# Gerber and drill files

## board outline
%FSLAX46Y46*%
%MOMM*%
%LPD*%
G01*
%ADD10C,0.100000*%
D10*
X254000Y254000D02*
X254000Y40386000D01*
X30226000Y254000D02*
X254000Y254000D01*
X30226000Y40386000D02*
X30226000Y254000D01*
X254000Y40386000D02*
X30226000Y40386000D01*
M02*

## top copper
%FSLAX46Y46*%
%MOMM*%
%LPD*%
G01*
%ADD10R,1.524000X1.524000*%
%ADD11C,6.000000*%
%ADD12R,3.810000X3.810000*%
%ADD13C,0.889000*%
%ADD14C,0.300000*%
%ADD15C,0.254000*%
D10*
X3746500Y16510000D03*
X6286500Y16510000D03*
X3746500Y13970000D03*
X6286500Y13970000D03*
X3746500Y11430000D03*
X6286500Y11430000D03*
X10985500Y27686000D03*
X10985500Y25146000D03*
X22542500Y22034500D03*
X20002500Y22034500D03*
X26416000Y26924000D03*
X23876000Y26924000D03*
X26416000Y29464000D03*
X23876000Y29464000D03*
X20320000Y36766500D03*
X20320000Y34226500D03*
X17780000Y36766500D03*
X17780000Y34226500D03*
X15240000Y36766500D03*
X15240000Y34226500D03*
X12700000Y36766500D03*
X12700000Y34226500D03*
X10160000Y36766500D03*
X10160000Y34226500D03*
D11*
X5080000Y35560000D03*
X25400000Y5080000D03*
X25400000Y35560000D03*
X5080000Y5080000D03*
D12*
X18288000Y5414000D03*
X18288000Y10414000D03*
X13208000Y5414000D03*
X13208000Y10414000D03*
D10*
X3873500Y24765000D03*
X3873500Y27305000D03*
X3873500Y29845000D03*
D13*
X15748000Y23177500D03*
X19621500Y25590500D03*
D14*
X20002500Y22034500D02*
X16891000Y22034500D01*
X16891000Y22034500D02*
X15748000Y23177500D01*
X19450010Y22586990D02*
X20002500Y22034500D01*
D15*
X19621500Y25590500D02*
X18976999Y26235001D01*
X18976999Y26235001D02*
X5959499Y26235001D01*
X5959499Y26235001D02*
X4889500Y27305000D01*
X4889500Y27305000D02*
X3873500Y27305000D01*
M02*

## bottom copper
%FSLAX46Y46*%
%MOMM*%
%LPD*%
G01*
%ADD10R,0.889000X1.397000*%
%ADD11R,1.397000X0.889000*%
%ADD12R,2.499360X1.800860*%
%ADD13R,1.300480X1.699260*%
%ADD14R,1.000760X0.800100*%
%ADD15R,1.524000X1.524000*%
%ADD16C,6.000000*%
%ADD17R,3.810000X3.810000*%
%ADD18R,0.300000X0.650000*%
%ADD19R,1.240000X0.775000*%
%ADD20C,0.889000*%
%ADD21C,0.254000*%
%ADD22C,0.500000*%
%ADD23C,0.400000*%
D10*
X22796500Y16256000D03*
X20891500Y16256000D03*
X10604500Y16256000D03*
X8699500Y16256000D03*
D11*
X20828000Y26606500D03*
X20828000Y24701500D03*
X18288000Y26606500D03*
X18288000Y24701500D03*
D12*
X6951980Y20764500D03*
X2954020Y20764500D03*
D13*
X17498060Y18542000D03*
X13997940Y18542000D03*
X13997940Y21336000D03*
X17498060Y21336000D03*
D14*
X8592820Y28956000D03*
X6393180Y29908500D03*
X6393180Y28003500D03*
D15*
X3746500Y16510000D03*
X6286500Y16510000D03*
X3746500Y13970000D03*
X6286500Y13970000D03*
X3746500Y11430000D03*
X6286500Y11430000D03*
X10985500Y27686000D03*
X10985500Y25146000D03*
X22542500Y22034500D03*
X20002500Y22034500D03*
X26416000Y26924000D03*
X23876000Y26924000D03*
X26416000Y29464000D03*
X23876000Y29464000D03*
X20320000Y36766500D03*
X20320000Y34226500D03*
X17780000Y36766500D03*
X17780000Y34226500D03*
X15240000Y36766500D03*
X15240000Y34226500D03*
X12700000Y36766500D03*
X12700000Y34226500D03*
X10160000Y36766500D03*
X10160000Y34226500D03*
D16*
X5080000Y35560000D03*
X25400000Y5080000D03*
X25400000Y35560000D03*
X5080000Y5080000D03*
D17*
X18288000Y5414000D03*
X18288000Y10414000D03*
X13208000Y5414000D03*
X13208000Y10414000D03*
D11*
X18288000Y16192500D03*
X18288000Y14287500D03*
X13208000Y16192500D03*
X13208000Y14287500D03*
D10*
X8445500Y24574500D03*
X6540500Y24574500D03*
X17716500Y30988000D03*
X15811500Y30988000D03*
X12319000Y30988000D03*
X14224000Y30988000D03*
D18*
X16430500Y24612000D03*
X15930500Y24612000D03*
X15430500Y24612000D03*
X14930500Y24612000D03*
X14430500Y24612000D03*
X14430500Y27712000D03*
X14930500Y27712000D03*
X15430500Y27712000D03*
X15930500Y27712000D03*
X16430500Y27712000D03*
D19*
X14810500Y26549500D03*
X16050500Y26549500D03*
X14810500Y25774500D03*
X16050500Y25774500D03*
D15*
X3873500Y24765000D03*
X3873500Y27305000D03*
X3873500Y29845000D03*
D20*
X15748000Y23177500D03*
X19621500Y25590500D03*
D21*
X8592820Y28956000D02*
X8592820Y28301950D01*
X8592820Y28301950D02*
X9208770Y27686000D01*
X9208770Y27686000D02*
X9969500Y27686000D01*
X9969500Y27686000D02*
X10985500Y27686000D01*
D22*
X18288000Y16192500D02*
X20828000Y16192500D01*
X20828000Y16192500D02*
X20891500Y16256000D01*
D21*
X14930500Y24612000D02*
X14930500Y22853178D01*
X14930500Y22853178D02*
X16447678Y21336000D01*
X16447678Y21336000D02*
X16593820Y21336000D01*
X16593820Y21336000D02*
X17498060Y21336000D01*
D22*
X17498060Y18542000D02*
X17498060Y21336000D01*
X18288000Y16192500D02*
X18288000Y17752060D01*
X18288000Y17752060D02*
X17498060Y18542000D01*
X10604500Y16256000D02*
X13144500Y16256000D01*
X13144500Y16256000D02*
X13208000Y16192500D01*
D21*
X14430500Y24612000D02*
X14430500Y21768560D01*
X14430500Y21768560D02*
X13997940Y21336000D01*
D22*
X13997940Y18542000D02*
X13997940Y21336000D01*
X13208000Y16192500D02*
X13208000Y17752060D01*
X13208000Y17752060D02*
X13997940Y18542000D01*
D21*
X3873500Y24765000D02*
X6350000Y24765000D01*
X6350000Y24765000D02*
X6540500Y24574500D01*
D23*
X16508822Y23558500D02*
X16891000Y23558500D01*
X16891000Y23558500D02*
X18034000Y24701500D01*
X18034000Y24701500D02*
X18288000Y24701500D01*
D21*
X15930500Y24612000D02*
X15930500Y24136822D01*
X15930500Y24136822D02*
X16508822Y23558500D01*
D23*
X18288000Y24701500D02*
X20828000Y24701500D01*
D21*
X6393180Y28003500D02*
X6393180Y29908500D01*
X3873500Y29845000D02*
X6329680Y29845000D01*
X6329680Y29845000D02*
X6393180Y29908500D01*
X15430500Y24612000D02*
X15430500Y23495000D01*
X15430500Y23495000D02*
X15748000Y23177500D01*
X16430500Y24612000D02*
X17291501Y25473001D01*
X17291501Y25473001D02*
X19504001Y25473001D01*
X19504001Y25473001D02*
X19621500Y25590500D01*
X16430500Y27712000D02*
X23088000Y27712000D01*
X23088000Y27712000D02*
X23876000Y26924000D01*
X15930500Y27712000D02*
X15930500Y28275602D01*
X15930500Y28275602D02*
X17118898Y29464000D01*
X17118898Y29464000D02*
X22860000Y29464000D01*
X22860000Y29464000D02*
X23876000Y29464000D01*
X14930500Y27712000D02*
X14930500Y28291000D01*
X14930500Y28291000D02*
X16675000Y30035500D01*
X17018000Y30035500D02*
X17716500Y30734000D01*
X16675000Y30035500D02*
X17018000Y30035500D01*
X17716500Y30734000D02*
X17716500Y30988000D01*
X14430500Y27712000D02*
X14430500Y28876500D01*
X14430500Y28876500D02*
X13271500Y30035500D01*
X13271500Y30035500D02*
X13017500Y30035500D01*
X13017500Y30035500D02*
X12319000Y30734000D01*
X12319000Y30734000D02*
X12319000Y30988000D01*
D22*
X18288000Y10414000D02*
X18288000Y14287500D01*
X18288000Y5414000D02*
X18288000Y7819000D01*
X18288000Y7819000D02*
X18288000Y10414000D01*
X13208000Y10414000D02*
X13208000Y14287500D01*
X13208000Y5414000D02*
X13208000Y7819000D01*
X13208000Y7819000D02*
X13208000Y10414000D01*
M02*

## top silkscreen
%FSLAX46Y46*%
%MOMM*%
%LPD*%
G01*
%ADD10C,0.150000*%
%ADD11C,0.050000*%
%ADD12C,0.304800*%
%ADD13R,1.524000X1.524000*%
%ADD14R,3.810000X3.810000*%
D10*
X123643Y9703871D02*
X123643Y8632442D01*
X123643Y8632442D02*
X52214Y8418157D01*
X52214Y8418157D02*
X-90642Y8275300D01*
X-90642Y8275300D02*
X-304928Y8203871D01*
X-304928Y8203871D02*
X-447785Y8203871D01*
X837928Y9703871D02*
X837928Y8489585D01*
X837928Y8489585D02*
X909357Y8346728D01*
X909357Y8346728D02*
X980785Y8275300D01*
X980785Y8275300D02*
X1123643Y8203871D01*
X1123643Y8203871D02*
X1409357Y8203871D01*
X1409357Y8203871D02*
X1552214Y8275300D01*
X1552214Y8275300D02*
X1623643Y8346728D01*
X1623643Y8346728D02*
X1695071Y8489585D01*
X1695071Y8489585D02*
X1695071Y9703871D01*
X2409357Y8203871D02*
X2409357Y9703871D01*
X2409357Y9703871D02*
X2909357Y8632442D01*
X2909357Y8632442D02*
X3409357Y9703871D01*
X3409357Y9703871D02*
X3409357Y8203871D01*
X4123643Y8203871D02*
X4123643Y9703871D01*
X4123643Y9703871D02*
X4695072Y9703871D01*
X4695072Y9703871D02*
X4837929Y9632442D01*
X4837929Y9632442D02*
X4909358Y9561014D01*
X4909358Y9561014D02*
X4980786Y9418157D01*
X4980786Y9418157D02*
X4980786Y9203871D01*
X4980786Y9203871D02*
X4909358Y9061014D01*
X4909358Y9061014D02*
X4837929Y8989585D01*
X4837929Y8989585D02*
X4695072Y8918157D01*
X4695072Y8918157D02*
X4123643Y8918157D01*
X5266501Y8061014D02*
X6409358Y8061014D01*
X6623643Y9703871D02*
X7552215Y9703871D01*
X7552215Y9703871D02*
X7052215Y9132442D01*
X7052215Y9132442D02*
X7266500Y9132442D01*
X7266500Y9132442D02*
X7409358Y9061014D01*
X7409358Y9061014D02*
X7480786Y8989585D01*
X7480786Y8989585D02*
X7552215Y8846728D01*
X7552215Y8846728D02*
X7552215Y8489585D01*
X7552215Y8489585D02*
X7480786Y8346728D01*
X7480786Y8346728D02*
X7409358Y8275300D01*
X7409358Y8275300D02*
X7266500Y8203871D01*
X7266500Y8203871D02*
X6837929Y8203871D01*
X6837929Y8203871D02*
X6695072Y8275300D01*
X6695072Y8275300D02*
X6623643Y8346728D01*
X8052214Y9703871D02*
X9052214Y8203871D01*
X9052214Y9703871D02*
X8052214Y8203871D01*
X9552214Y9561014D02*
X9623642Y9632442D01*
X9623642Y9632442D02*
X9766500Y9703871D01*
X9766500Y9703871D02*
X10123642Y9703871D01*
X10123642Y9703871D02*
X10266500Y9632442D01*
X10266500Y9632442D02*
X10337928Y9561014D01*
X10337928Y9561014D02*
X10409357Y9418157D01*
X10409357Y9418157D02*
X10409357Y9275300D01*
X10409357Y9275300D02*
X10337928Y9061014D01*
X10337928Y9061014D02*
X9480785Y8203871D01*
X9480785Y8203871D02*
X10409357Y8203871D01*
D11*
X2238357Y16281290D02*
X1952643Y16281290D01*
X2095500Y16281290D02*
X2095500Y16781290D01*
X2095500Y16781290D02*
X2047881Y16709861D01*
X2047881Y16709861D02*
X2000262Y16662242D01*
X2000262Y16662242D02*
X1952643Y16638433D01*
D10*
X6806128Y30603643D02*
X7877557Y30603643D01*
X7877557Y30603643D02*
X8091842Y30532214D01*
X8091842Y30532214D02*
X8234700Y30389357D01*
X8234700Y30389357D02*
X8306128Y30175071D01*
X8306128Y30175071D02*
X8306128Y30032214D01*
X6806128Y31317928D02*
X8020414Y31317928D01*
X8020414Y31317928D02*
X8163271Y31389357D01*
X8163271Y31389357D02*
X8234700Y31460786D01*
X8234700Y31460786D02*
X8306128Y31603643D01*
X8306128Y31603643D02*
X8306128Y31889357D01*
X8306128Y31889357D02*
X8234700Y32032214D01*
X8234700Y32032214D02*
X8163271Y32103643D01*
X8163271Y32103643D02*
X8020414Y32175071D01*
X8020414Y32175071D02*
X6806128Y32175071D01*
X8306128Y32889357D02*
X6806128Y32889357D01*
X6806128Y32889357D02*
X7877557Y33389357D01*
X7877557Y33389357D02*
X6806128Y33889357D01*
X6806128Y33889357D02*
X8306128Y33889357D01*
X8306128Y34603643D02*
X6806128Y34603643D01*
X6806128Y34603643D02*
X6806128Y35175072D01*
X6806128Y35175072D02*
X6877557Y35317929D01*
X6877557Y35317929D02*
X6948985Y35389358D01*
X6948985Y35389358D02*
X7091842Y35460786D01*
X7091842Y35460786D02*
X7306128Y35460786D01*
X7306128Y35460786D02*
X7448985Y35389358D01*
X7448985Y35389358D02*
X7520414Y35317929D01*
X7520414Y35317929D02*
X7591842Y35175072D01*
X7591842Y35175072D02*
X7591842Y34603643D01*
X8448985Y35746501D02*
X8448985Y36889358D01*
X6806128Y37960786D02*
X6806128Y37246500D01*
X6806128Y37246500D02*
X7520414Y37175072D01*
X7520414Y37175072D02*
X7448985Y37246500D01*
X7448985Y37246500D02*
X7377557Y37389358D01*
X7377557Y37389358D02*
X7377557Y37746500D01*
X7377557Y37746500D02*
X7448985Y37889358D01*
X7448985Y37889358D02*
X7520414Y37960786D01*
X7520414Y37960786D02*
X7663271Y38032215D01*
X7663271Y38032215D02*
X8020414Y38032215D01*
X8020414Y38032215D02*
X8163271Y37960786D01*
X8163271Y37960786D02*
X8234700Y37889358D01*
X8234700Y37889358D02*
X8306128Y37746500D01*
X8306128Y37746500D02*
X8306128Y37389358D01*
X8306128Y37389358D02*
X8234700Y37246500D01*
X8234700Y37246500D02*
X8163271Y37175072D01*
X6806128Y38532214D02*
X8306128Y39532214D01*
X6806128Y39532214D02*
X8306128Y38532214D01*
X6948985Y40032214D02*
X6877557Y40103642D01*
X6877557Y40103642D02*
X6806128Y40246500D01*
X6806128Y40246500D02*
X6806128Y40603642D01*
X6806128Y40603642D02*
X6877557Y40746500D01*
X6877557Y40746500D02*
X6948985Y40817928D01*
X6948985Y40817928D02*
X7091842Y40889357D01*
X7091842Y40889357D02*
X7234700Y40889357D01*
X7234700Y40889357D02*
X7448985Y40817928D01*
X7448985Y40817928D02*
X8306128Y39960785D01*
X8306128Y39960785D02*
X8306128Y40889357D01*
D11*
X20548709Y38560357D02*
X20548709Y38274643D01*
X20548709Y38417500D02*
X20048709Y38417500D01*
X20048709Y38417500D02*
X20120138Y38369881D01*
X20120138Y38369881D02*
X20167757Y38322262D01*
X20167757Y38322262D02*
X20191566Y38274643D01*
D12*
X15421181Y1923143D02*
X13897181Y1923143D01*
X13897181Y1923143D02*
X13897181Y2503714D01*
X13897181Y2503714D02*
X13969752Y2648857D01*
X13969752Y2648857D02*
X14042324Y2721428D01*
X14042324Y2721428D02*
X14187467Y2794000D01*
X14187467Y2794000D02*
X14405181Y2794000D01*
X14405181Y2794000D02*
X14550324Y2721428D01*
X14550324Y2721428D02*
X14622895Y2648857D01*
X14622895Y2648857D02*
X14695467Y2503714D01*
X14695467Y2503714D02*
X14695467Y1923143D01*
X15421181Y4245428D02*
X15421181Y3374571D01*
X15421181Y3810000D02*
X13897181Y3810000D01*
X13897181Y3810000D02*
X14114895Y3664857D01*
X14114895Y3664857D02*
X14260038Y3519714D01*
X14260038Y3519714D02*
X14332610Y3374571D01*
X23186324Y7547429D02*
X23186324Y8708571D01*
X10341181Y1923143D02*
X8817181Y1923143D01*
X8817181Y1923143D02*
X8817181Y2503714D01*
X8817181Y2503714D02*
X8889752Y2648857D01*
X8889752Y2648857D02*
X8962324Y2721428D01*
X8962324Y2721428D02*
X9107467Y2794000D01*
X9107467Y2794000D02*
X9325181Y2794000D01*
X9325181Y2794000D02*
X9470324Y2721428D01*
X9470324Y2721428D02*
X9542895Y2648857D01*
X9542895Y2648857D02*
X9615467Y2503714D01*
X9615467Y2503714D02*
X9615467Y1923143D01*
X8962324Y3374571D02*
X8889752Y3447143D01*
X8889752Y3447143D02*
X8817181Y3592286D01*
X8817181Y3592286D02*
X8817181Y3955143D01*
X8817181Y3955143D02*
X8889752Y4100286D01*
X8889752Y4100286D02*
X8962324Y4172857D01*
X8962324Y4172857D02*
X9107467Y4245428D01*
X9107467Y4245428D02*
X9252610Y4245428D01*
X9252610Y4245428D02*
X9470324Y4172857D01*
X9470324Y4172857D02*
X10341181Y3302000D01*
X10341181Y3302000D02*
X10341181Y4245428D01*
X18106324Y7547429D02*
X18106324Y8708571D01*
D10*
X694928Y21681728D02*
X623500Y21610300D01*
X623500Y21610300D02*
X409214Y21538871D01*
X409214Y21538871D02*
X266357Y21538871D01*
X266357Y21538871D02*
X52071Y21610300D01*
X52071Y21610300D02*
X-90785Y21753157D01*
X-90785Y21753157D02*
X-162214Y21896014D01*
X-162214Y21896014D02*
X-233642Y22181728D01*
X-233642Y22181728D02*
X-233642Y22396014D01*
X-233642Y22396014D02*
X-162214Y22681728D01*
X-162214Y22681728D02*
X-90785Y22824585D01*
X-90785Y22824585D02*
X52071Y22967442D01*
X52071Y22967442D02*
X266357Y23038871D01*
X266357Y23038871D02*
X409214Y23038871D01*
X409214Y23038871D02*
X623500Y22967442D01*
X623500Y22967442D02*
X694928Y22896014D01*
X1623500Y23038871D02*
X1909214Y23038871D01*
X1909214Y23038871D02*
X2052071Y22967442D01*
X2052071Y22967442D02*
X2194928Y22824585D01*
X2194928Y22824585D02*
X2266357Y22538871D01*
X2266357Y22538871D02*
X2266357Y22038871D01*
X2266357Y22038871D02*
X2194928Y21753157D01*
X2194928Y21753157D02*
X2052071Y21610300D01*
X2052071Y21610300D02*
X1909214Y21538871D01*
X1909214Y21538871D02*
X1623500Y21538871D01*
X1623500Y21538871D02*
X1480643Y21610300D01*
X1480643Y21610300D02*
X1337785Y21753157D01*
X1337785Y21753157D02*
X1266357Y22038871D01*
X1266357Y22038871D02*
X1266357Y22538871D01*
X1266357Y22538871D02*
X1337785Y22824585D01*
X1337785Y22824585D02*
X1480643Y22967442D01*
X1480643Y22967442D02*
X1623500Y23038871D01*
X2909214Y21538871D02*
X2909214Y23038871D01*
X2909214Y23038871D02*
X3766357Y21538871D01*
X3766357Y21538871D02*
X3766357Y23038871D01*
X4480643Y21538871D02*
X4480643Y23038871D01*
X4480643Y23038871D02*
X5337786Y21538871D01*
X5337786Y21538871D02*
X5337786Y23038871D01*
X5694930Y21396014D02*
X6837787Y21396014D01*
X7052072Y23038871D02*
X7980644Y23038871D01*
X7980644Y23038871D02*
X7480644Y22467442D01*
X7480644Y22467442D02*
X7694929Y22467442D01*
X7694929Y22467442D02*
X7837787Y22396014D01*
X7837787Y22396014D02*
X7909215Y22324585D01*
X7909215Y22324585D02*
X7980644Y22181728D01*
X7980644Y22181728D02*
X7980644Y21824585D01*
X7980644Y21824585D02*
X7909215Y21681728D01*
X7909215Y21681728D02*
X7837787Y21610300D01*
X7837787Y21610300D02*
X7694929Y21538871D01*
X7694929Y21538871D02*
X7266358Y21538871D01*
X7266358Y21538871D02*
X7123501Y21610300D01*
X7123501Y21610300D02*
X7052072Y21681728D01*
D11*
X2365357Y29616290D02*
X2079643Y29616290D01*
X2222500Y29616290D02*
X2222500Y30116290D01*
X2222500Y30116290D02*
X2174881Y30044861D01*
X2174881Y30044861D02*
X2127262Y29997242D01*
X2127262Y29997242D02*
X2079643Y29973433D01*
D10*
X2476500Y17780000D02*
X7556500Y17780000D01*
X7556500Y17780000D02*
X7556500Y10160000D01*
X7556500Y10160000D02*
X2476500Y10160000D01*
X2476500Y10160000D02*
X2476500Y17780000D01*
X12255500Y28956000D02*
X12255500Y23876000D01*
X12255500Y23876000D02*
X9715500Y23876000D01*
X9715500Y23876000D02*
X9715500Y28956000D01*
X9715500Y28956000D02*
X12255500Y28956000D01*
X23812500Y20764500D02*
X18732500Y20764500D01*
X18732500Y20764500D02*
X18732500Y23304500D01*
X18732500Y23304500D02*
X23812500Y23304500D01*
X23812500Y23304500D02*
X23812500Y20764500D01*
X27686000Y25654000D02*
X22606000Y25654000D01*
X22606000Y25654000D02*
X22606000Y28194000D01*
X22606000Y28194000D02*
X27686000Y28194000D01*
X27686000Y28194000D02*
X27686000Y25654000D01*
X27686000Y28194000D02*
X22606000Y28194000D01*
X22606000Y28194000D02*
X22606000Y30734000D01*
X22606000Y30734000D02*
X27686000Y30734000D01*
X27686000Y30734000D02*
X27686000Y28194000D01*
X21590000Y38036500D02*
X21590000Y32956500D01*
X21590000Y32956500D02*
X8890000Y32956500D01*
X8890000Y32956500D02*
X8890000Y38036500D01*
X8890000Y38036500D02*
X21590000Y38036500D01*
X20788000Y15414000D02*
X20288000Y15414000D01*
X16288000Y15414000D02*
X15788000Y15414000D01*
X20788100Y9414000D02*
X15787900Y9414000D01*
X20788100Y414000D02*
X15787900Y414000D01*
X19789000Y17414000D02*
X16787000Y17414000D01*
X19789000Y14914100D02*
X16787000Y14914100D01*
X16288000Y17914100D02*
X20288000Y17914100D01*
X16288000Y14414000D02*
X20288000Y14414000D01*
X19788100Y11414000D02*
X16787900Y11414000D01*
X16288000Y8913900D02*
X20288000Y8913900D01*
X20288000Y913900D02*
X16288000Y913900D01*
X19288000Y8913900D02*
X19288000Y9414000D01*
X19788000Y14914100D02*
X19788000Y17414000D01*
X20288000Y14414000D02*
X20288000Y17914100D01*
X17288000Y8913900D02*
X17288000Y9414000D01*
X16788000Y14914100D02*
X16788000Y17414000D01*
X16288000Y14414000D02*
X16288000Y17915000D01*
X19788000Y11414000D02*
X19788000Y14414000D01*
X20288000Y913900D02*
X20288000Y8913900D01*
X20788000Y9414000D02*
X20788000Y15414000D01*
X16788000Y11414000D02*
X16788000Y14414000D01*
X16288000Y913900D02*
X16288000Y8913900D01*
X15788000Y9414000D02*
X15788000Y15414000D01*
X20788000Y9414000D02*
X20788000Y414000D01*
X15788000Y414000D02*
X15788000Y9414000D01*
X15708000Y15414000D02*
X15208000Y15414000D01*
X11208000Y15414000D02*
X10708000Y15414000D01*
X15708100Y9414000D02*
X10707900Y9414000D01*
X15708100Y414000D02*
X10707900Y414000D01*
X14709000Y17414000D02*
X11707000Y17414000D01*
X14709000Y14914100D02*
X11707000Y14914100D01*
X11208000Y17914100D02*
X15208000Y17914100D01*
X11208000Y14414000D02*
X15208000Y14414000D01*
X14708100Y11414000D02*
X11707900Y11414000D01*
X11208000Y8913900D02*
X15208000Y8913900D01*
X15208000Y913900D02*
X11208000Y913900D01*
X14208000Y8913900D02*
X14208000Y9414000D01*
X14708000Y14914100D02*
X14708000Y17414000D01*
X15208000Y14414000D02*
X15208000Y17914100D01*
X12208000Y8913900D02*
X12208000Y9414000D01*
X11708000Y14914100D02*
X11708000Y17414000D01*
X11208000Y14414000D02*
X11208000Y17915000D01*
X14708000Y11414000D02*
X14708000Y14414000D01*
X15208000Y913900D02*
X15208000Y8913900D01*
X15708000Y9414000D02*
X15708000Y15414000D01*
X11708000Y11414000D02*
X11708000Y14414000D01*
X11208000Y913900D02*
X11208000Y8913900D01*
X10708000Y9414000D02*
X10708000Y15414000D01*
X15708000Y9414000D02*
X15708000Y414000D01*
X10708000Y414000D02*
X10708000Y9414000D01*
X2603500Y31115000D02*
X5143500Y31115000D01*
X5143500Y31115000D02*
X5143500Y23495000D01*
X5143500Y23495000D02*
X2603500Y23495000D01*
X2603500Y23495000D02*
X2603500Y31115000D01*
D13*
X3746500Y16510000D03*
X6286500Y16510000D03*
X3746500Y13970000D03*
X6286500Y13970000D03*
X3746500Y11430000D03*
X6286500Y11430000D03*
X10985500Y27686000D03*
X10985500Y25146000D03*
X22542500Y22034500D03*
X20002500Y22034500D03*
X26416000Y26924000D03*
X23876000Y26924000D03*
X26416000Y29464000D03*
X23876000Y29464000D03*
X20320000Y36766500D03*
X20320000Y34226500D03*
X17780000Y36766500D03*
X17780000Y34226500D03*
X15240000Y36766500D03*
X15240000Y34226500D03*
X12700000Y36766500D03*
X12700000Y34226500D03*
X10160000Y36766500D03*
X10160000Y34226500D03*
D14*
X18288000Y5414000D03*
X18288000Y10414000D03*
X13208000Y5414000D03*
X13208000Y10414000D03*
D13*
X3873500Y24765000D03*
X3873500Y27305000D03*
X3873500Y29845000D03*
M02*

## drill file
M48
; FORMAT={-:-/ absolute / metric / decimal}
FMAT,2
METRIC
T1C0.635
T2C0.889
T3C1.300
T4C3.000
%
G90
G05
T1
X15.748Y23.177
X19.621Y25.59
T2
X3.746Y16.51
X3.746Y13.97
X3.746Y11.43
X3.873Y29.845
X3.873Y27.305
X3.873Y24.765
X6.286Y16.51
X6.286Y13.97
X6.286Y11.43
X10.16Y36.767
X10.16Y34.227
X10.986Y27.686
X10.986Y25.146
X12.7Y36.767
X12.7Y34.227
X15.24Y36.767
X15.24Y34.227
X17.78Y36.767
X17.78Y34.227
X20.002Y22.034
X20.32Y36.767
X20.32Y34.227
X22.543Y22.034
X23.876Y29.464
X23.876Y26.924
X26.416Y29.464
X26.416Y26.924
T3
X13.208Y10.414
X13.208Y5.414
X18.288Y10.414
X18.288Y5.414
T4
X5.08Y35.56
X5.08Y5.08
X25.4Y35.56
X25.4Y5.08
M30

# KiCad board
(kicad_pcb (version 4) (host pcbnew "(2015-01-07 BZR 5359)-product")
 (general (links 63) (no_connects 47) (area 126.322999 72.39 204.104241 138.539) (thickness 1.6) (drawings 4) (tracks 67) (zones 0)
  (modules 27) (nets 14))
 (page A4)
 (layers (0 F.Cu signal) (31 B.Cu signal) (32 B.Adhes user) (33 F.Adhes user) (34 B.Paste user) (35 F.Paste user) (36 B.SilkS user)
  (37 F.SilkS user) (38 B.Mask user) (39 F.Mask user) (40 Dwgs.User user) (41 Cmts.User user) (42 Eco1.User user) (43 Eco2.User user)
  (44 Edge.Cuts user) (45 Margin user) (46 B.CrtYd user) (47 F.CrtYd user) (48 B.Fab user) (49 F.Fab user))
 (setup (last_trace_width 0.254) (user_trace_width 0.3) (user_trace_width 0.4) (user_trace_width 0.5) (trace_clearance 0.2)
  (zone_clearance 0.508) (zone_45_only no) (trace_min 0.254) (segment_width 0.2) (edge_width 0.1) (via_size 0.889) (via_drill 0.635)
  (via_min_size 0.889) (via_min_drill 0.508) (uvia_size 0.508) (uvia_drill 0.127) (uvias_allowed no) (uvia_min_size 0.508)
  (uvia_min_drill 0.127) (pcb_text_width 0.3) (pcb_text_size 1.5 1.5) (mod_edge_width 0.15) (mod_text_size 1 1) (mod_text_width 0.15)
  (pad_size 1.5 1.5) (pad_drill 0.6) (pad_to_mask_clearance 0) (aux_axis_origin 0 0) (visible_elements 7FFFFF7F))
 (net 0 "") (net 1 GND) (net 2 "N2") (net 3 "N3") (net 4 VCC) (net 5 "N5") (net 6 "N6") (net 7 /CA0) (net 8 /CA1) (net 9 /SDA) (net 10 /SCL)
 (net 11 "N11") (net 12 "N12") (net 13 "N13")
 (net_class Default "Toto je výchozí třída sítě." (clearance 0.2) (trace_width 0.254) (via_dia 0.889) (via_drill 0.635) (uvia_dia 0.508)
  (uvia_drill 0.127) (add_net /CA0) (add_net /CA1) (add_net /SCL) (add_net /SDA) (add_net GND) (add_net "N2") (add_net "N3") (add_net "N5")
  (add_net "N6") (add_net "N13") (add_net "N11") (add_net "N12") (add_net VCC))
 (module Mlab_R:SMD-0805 (layer B.Cu) (at 21.844 -16.256 180)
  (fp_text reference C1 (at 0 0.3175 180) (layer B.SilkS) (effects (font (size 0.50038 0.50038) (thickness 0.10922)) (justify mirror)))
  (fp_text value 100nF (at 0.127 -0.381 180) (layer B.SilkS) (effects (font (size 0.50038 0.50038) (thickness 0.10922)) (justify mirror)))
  (pad 1 smd rect (at -0.9525 0 180) (size 0.889 1.397) (layers B.Cu B.Paste B.Mask) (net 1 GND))
  (pad 2 smd rect (at 0.9525 0 180) (size 0.889 1.397) (layers B.Cu B.Paste B.Mask) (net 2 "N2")))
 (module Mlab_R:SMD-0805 (layer B.Cu) (at 9.652 -16.256 180)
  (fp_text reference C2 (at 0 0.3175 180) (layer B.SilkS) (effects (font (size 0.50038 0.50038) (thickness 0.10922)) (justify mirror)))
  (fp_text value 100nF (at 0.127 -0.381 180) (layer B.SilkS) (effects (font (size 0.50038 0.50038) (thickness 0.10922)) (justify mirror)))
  (pad 1 smd rect (at -0.9525 0 180) (size 0.889 1.397) (layers B.Cu B.Paste B.Mask) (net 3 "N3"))
  (pad 2 smd rect (at 0.9525 0 180) (size 0.889 1.397) (layers B.Cu B.Paste B.Mask) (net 1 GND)))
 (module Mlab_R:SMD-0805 (layer B.Cu) (at 20.828 -25.654 270)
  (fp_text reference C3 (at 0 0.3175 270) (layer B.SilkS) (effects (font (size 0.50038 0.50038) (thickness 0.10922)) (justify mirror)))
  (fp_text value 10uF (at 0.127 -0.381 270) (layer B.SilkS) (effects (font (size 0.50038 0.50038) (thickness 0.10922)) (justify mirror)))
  (pad 1 smd rect (at -0.9525 0 270) (size 0.889 1.397) (layers B.Cu B.Paste B.Mask) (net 1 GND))
  (pad 2 smd rect (at 0.9525 0 270) (size 0.889 1.397) (layers B.Cu B.Paste B.Mask) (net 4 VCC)))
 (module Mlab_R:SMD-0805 (layer B.Cu) (at 18.288 -25.654 270)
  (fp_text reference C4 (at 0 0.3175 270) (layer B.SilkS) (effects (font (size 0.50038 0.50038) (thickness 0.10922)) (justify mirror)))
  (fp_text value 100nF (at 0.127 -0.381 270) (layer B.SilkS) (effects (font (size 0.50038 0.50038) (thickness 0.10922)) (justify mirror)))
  (pad 1 smd rect (at -0.9525 0 270) (size 0.889 1.397) (layers B.Cu B.Paste B.Mask) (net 1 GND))
  (pad 2 smd rect (at 0.9525 0 270) (size 0.889 1.397) (layers B.Cu B.Paste B.Mask) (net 4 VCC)))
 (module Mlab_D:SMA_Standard (layer B.Cu) (at 4.953 -20.7645 180)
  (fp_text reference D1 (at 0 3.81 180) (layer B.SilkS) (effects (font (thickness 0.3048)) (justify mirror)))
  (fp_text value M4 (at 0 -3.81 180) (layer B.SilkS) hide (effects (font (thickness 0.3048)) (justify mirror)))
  (pad 1 smd rect (at -1.99898 0 180) (size 2.49936 1.80086) (layers B.Cu B.Paste B.Mask) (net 1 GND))
  (pad 2 smd rect (at 1.99898 0 180) (size 2.49936 1.80086) (layers B.Cu B.Paste B.Mask) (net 4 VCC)))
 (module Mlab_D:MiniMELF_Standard (layer B.Cu) (at 15.748 -18.542 180)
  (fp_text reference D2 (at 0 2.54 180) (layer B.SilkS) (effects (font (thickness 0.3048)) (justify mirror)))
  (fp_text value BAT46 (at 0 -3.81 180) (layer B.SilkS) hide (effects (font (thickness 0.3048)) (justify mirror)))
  (pad 1 smd rect (at -1.75006 0 180) (size 1.30048 1.69926) (layers B.Cu B.Paste B.Mask) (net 2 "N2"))
  (pad 2 smd rect (at 1.75006 0 180) (size 1.30048 1.69926) (layers B.Cu B.Paste B.Mask) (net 3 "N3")))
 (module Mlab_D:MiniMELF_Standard (layer B.Cu) (at 15.748 -21.336)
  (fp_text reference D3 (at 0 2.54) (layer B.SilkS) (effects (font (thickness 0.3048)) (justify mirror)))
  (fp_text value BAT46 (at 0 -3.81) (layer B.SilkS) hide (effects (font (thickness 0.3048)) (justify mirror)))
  (pad 1 smd rect (at -1.75006 0) (size 1.30048 1.69926) (layers B.Cu B.Paste B.Mask) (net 3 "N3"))
  (pad 2 smd rect (at 1.75006 0) (size 1.30048 1.69926) (layers B.Cu B.Paste B.Mask) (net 2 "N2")))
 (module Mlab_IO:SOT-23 (layer B.Cu) (at 7.493 -28.956 90)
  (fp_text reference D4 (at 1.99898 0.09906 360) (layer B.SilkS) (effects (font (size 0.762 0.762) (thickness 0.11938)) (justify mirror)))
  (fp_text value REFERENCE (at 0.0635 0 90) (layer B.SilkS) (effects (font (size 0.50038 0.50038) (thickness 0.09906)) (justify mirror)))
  (pad 3 smd rect (at 0 1.09982 90) (size 0.8001 1.00076) (layers B.Cu B.Paste B.Mask) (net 1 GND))
  (pad 2 smd rect (at 0.9525 -1.09982 90) (size 0.8001 1.00076) (layers B.Cu B.Paste B.Mask) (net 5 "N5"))
  (pad 1 smd rect (at -0.9525 -1.09982 90) (size 0.8001 1.00076) (layers B.Cu B.Paste B.Mask) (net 5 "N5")))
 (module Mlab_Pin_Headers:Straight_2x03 (layer F.Cu) (at 5.0165 -13.97)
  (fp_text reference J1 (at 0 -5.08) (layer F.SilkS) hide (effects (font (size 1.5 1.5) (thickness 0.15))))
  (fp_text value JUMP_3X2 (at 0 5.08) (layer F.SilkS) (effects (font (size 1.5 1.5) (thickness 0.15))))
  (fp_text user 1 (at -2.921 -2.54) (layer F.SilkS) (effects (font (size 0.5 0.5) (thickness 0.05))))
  (fp_line (start -2.54 -3.81) (end 2.54 -3.81) (layer F.SilkS) (width 0.15))
  (fp_line (start 2.54 -3.81) (end 2.54 3.81) (layer F.SilkS) (width 0.15))
  (fp_line (start 2.54 3.81) (end -2.54 3.81) (layer F.SilkS) (width 0.15))
  (fp_line (start -2.54 3.81) (end -2.54 -3.81) (layer F.SilkS) (width 0.15))
  (pad 1 thru_hole rect (at -1.27 -2.54) (size 1.524 1.524) (drill 0.889) (layers *.Cu *.Mask F.SilkS) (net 1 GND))
  (pad 2 thru_hole rect (at 1.27 -2.54) (size 1.524 1.524) (drill 0.889) (layers *.Cu *.Mask F.SilkS) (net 1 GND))
  (pad 3 thru_hole rect (at -1.27 0) (size 1.524 1.524) (drill 0.889) (layers *.Cu *.Mask F.SilkS) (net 4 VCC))
  (pad 4 thru_hole rect (at 1.27 0) (size 1.524 1.524) (drill 0.889) (layers *.Cu *.Mask F.SilkS) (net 4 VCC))
  (pad 5 thru_hole rect (at -1.27 2.54) (size 1.524 1.524) (drill 0.889) (layers *.Cu *.Mask F.SilkS) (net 1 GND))
  (pad 6 thru_hole rect (at 1.27 2.54) (size 1.524 1.524) (drill 0.889) (layers *.Cu *.Mask F.SilkS) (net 1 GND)))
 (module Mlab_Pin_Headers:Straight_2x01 (layer F.Cu) (at 10.9855 -26.416 270)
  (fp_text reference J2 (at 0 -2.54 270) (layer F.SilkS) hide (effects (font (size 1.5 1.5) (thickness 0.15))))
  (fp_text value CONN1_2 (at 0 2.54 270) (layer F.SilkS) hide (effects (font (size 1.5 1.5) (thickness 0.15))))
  (fp_line (start -2.54 -1.27) (end 2.54 -1.27) (layer F.SilkS) (width 0.15))
  (fp_line (start 2.54 -1.27) (end 2.54 1.27) (layer F.SilkS) (width 0.15))
  (fp_line (start 2.54 1.27) (end -2.54 1.27) (layer F.SilkS) (width 0.15))
  (fp_line (start -2.54 1.27) (end -2.54 -1.27) (layer F.SilkS) (width 0.15))
  (pad 1 thru_hole rect (at -1.27 0 270) (size 1.524 1.524) (drill 0.889) (layers *.Cu *.Mask F.SilkS) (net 1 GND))
  (pad 2 thru_hole rect (at 1.27 0 270) (size 1.524 1.524) (drill 0.889) (layers *.Cu *.Mask F.SilkS) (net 3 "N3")))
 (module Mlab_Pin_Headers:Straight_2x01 (layer F.Cu) (at 21.2725 -22.0345 180)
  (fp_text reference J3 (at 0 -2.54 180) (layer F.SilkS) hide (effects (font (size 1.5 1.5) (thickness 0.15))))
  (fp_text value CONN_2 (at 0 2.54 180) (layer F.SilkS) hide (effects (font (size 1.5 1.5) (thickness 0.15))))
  (fp_line (start -2.54 -1.27) (end 2.54 -1.27) (layer F.SilkS) (width 0.15))
  (fp_line (start 2.54 -1.27) (end 2.54 1.27) (layer F.SilkS) (width 0.15))
  (fp_line (start 2.54 1.27) (end -2.54 1.27) (layer F.SilkS) (width 0.15))
  (fp_line (start -2.54 1.27) (end -2.54 -1.27) (layer F.SilkS) (width 0.15))
  (pad 1 thru_hole rect (at -1.27 0 180) (size 1.524 1.524) (drill 0.889) (layers *.Cu *.Mask F.SilkS) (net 1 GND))
  (pad 2 thru_hole rect (at 1.27 0 180) (size 1.524 1.524) (drill 0.889) (layers *.Cu *.Mask F.SilkS) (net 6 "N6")))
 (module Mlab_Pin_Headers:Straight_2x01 (layer F.Cu) (at 25.146 -26.924 180)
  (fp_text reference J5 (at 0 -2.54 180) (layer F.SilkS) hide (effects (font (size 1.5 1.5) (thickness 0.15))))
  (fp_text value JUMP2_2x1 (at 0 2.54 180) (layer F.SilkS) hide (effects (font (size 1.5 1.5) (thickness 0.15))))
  (fp_line (start -2.54 -1.27) (end 2.54 -1.27) (layer F.SilkS) (width 0.15))
  (fp_line (start 2.54 -1.27) (end 2.54 1.27) (layer F.SilkS) (width 0.15))
  (fp_line (start 2.54 1.27) (end -2.54 1.27) (layer F.SilkS) (width 0.15))
  (fp_line (start -2.54 1.27) (end -2.54 -1.27) (layer F.SilkS) (width 0.15))
  (pad 1 thru_hole rect (at -1.27 0 180) (size 1.524 1.524) (drill 0.889) (layers *.Cu *.Mask F.SilkS) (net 4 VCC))
  (pad 2 thru_hole rect (at 1.27 0 180) (size 1.524 1.524) (drill 0.889) (layers *.Cu *.Mask F.SilkS) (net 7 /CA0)))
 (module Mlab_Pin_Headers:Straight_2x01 (layer F.Cu) (at 25.146 -29.464 180)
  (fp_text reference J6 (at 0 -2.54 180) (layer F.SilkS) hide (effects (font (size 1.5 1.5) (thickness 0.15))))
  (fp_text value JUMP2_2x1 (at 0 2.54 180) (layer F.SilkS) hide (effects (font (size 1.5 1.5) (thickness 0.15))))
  (fp_line (start -2.54 -1.27) (end 2.54 -1.27) (layer F.SilkS) (width 0.15))
  (fp_line (start 2.54 -1.27) (end 2.54 1.27) (layer F.SilkS) (width 0.15))
  (fp_line (start 2.54 1.27) (end -2.54 1.27) (layer F.SilkS) (width 0.15))
  (fp_line (start -2.54 1.27) (end -2.54 -1.27) (layer F.SilkS) (width 0.15))
  (pad 1 thru_hole rect (at -1.27 0 180) (size 1.524 1.524) (drill 0.889) (layers *.Cu *.Mask F.SilkS) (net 4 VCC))
  (pad 2 thru_hole rect (at 1.27 0 180) (size 1.524 1.524) (drill 0.889) (layers *.Cu *.Mask F.SilkS) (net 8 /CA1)))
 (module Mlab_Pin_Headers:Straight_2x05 (layer F.Cu) (at 15.24 -35.4965 270)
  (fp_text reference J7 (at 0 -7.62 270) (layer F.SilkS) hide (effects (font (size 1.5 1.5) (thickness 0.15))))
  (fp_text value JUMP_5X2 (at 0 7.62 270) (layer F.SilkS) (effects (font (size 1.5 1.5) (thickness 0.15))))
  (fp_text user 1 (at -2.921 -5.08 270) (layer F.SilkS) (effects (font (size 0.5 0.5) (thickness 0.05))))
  (fp_line (start -2.54 -6.35) (end 2.54 -6.35) (layer F.SilkS) (width 0.15))
  (fp_line (start 2.54 -6.35) (end 2.54 6.35) (layer F.SilkS) (width 0.15))
  (fp_line (start 2.54 6.35) (end -2.54 6.35) (layer F.SilkS) (width 0.15))
  (fp_line (start -2.54 6.35) (end -2.54 -6.35) (layer F.SilkS) (width 0.15))
  (pad 1 thru_hole rect (at -1.27 -5.08 270) (size 1.524 1.524) (drill 0.889) (layers *.Cu *.Mask F.SilkS) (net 1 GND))
  (pad 2 thru_hole rect (at 1.27 -5.08 270) (size 1.524 1.524) (drill 0.889) (layers *.Cu *.Mask F.SilkS) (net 1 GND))
  (pad 3 thru_hole rect (at -1.27 -2.54 270) (size 1.524 1.524) (drill 0.889) (layers *.Cu *.Mask F.SilkS) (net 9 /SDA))
  (pad 4 thru_hole rect (at 1.27 -2.54 270) (size 1.524 1.524) (drill 0.889) (layers *.Cu *.Mask F.SilkS) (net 9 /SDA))
  (pad 5 thru_hole rect (at -1.27 0 270) (size 1.524 1.524) (drill 0.889) (layers *.Cu *.Mask F.SilkS) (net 4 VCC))
  (pad 6 thru_hole rect (at 1.27 0 270) (size 1.524 1.524) (drill 0.889) (layers *.Cu *.Mask F.SilkS) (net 4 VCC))
  (pad 7 thru_hole rect (at -1.27 2.54 270) (size 1.524 1.524) (drill 0.889) (layers *.Cu *.Mask F.SilkS) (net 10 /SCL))
  (pad 8 thru_hole rect (at 1.27 2.54 270) (size 1.524 1.524) (drill 0.889) (layers *.Cu *.Mask F.SilkS) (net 10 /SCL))
  (pad 9 thru_hole rect (at -1.27 5.08 270) (size 1.524 1.524) (drill 0.889) (layers *.Cu *.Mask F.SilkS) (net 1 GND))
  (pad 10 thru_hole rect (at 1.27 5.08 270) (size 1.524 1.524) (drill 0.889) (layers *.Cu *.Mask F.SilkS) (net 1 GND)))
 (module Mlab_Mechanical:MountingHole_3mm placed (layer F.Cu) (at 5.08 -35.56)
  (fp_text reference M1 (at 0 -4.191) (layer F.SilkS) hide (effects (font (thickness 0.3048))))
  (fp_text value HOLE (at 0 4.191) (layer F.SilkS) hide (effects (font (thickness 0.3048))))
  (pad 1 thru_hole circle (at 0 0) (size 6 6) (drill 3) (layers *.Cu *.Adhes *.Mask) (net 1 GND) (clearance 1) (zone_connect 2)))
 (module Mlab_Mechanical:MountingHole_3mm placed (layer F.Cu) (at 25.4 -5.08)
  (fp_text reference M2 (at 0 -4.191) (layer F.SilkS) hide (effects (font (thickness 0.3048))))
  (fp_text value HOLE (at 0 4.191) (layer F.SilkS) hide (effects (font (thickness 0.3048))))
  (pad 1 thru_hole circle (at 0 0) (size 6 6) (drill 3) (layers *.Cu *.Adhes *.Mask) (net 1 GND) (clearance 1) (zone_connect 2)))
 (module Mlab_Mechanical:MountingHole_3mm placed (layer F.Cu) (at 25.4 -35.56)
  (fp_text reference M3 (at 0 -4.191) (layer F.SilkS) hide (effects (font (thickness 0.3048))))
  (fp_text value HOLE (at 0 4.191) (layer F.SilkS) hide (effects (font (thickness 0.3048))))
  (pad 1 thru_hole circle (at 0 0) (size 6 6) (drill 3) (layers *.Cu *.Adhes *.Mask) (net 1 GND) (clearance 1) (zone_connect 2)))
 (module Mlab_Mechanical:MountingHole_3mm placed (layer F.Cu) (at 5.08 -5.08)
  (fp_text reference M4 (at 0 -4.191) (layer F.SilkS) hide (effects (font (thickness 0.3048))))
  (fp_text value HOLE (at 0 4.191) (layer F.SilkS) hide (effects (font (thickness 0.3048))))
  (pad 1 thru_hole circle (at 0 0) (size 6 6) (drill 3) (layers *.Cu *.Adhes *.Mask) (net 1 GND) (clearance 1) (zone_connect 2)))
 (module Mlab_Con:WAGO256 (layer F.Cu) (at 18.288 -7.874 90)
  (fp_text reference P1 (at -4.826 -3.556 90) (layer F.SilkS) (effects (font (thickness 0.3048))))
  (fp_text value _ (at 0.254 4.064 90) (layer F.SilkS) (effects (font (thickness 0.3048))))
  (fp_line (start 7.54 2.5) (end 7.54 2) (layer F.SilkS) (width 0.15))
  (fp_line (start 7.54 -2) (end 7.54 -2.5) (layer F.SilkS) (width 0.15))
  (fp_line (start 1.54 2.5001) (end 1.54 -2.5001) (layer F.SilkS) (width 0.15))
  (fp_line (start -7.46 2.5001) (end -7.46 -2.5001) (layer F.SilkS) (width 0.15))
  (fp_line (start 9.54 1.501) (end 9.54 -1.501) (layer F.SilkS) (width 0.15))
  (fp_line (start 7.0401 1.501) (end 7.0401 -1.501) (layer F.SilkS) (width 0.15))
  (fp_line (start 10.0401 -2) (end 10.0401 2) (layer F.SilkS) (width 0.15))
  (fp_line (start 6.54 -2) (end 6.54 2) (layer F.SilkS) (width 0.15))
  (fp_line (start 3.54 1.5001) (end 3.54 -1.5001) (layer F.SilkS) (width 0.15))
  (fp_line (start 1.0399 -2) (end 1.0399 2) (layer F.SilkS) (width 0.15))
  (fp_line (start -6.9601 2) (end -6.9601 -2) (layer F.SilkS) (width 0.15))
  (fp_line (start 1.0399 1) (end 1.54 1) (layer F.SilkS) (width 0.15))
  (fp_line (start 7.0401 1.5) (end 9.54 1.5) (layer F.SilkS) (width 0.15))
  (fp_line (start 6.54 2) (end 10.0401 2) (layer F.SilkS) (width 0.15))
  (fp_line (start 1.0399 -1) (end 1.54 -1) (layer F.SilkS) (width 0.15))
  (fp_line (start 7.0401 -1.5) (end 9.54 -1.5) (layer F.SilkS) (width 0.15))
  (fp_line (start 6.54 -2) (end 10.041 -2) (layer F.SilkS) (width 0.15))
  (fp_line (start 3.54 1.5) (end 6.54 1.5) (layer F.SilkS) (width 0.15))
  (fp_line (start -6.9601 2) (end 1.0399 2) (layer F.SilkS) (width 0.15))
  (fp_line (start 1.54 2.5) (end 7.54 2.5) (layer F.SilkS) (width 0.15))
  (fp_line (start 3.54 -1.5) (end 6.54 -1.5) (layer F.SilkS) (width 0.15))
  (fp_line (start -6.9601 -2) (end 1.0399 -2) (layer F.SilkS) (width 0.15))
  (fp_line (start 1.54 -2.5) (end 7.54 -2.5) (layer F.SilkS) (width 0.15))
  (fp_line (start 1.54 2.5) (end -7.46 2.5) (layer F.SilkS) (width 0.15))
  (fp_line (start -7.46 -2.5) (end 1.54 -2.5) (layer F.SilkS) (width 0.15))
  (pad 1 thru_hole rect (at -2.46 0 180) (size 3.81 3.81) (drill 1.3) (layers *.Cu *.Mask F.SilkS) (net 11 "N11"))
  (pad 1 thru_hole rect (at 2.54 0 180) (size 3.81 3.81) (drill 1.3) (layers *.Cu *.Mask F.SilkS) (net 11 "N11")))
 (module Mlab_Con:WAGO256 (layer F.Cu) (at 13.208 -7.874 90)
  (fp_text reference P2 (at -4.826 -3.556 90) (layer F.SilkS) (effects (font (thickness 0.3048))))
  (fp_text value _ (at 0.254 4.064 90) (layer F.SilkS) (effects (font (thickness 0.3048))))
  (fp_line (start 7.54 2.5) (end 7.54 2) (layer F.SilkS) (width 0.15))
  (fp_line (start 7.54 -2) (end 7.54 -2.5) (layer F.SilkS) (width 0.15))
  (fp_line (start 1.54 2.5001) (end 1.54 -2.5001) (layer F.SilkS) (width 0.15))
  (fp_line (start -7.46 2.5001) (end -7.46 -2.5001) (layer F.SilkS) (width 0.15))
  (fp_line (start 9.54 1.501) (end 9.54 -1.501) (layer F.SilkS) (width 0.15))
  (fp_line (start 7.0401 1.501) (end 7.0401 -1.501) (layer F.SilkS) (width 0.15))
  (fp_line (start 10.0401 -2) (end 10.0401 2) (layer F.SilkS) (width 0.15))
  (fp_line (start 6.54 -2) (end 6.54 2) (layer F.SilkS) (width 0.15))
  (fp_line (start 3.54 1.5001) (end 3.54 -1.5001) (layer F.SilkS) (width 0.15))
  (fp_line (start 1.0399 -2) (end 1.0399 2) (layer F.SilkS) (width 0.15))
  (fp_line (start -6.9601 2) (end -6.9601 -2) (layer F.SilkS) (width 0.15))
  (fp_line (start 1.0399 1) (end 1.54 1) (layer F.SilkS) (width 0.15))
  (fp_line (start 7.0401 1.5) (end 9.54 1.5) (layer F.SilkS) (width 0.15))
  (fp_line (start 6.54 2) (end 10.0401 2) (layer F.SilkS) (width 0.15))
  (fp_line (start 1.0399 -1) (end 1.54 -1) (layer F.SilkS) (width 0.15))
  (fp_line (start 7.0401 -1.5) (end 9.54 -1.5) (layer F.SilkS) (width 0.15))
  (fp_line (start 6.54 -2) (end 10.041 -2) (layer F.SilkS) (width 0.15))
  (fp_line (start 3.54 1.5) (end 6.54 1.5) (layer F.SilkS) (width 0.15))
  (fp_line (start -6.9601 2) (end 1.0399 2) (layer F.SilkS) (width 0.15))
  (fp_line (start 1.54 2.5) (end 7.54 2.5) (layer F.SilkS) (width 0.15))
  (fp_line (start 3.54 -1.5) (end 6.54 -1.5) (layer F.SilkS) (width 0.15))
  (fp_line (start -6.9601 -2) (end 1.0399 -2) (layer F.SilkS) (width 0.15))
  (fp_line (start 1.54 -2.5) (end 7.54 -2.5) (layer F.SilkS) (width 0.15))
  (fp_line (start 1.54 2.5) (end -7.46 2.5) (layer F.SilkS) (width 0.15))
  (fp_line (start -7.46 -2.5) (end 1.54 -2.5) (layer F.SilkS) (width 0.15))
  (pad 1 thru_hole rect (at -2.46 0 180) (size 3.81 3.81) (drill 1.3) (layers *.Cu *.Mask F.SilkS) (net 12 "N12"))
  (pad 1 thru_hole rect (at 2.54 0 180) (size 3.81 3.81) (drill 1.3) (layers *.Cu *.Mask F.SilkS) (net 12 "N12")))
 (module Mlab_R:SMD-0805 (layer B.Cu) (at 18.288 -15.24 270)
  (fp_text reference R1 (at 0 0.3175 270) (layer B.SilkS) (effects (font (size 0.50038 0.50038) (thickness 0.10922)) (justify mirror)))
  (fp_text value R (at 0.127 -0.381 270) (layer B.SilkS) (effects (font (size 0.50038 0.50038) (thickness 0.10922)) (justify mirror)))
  (pad 1 smd rect (at -0.9525 0 270) (size 0.889 1.397) (layers B.Cu B.Paste B.Mask) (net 2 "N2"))
  (pad 2 smd rect (at 0.9525 0 270) (size 0.889 1.397) (layers B.Cu B.Paste B.Mask) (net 11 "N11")))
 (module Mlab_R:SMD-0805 (layer B.Cu) (at 13.208 -15.24 270)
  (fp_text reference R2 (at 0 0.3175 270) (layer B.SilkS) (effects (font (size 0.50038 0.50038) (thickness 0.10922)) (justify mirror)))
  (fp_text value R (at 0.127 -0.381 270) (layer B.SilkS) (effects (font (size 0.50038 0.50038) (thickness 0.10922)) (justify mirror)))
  (pad 1 smd rect (at -0.9525 0 270) (size 0.889 1.397) (layers B.Cu B.Paste B.Mask) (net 3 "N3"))
  (pad 2 smd rect (at 0.9525 0 270) (size 0.889 1.397) (layers B.Cu B.Paste B.Mask) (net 12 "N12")))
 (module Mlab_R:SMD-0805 (layer B.Cu) (at 7.493 -24.5745 180)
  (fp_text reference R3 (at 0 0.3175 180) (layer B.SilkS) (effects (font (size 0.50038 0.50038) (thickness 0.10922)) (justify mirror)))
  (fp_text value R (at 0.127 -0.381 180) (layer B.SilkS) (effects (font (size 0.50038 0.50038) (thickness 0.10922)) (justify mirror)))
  (pad 1 smd rect (at -0.9525 0 180) (size 0.889 1.397) (layers B.Cu B.Paste B.Mask) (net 5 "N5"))
  (pad 2 smd rect (at 0.9525 0 180) (size 0.889 1.397) (layers B.Cu B.Paste B.Mask) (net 4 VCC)))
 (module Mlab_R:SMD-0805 (layer B.Cu) (at 16.764 -30.988 180)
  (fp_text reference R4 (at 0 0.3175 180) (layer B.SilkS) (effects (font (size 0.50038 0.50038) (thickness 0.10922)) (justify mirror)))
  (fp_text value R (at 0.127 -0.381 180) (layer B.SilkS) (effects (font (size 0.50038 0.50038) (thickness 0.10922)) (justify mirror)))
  (pad 1 smd rect (at -0.9525 0 180) (size 0.889 1.397) (layers B.Cu B.Paste B.Mask) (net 9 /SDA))
  (pad 2 smd rect (at 0.9525 0 180) (size 0.889 1.397) (layers B.Cu B.Paste B.Mask) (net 4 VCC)))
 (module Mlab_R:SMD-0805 (layer B.Cu) (at 13.2715 -30.988)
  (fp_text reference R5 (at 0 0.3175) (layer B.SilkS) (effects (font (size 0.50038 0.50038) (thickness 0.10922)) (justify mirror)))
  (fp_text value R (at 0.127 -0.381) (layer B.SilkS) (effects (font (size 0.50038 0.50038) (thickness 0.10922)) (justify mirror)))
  (pad 1 smd rect (at -0.9525 0) (size 0.889 1.397) (layers B.Cu B.Paste B.Mask) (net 10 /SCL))
  (pad 2 smd rect (at 0.9525 0) (size 0.889 1.397) (layers B.Cu B.Paste B.Mask) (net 4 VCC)))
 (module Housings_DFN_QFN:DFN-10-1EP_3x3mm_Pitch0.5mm (layer B.Cu) (at 15.4305 -26.162 90)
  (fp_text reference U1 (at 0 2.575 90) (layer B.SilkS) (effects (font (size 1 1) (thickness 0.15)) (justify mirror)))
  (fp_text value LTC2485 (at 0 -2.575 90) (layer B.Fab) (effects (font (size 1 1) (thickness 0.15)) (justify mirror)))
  (pad 1 smd rect (at -1.55 1 90) (size 0.65 0.3) (layers B.Cu B.Paste B.Mask) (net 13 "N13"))
  (pad 2 smd rect (at -1.55 0.5 90) (size 0.65 0.3) (layers B.Cu B.Paste B.Mask) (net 4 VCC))
  (pad 3 smd rect (at -1.55 0 90) (size 0.65 0.3) (layers B.Cu B.Paste B.Mask) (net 6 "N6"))
  (pad 4 smd rect (at -1.55 -0.5 90) (size 0.65 0.3) (layers B.Cu B.Paste B.Mask) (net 2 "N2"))
  (pad 5 smd rect (at -1.55 -1 90) (size 0.65 0.3) (layers B.Cu B.Paste B.Mask) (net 3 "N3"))
  (pad 6 smd rect (at 1.55 -1 90) (size 0.65 0.3) (layers B.Cu B.Paste B.Mask) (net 10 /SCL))
  (pad 7 smd rect (at 1.55 -0.5 90) (size 0.65 0.3) (layers B.Cu B.Paste B.Mask) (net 9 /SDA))
  (pad 8 smd rect (at 1.55 0 90) (size 0.65 0.3) (layers B.Cu B.Paste B.Mask) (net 1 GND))
  (pad 9 smd rect (at 1.55 0.5 90) (size 0.65 0.3) (layers B.Cu B.Paste B.Mask) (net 8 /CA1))
  (pad 10 smd rect (at 1.55 1 90) (size 0.65 0.3) (layers B.Cu B.Paste B.Mask) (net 7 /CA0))
  (pad 11 smd rect (at 0.3875 -0.62 90) (size 0.775 1.24) (layers B.Cu B.Paste B.Mask) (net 1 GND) (solder_paste_margin_ratio -0.2))
  (pad 11 smd rect (at 0.3875 0.62 90) (size 0.775 1.24) (layers B.Cu B.Paste B.Mask) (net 1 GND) (solder_paste_margin_ratio -0.2))
  (pad 11 smd rect (at -0.3875 -0.62 90) (size 0.775 1.24) (layers B.Cu B.Paste B.Mask) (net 1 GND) (solder_paste_margin_ratio -0.2))
  (pad 11 smd rect (at -0.3875 0.62 90) (size 0.775 1.24) (layers B.Cu B.Paste B.Mask) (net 1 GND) (solder_paste_margin_ratio -0.2)))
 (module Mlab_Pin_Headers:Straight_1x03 (layer F.Cu) (at 3.8735 -27.305)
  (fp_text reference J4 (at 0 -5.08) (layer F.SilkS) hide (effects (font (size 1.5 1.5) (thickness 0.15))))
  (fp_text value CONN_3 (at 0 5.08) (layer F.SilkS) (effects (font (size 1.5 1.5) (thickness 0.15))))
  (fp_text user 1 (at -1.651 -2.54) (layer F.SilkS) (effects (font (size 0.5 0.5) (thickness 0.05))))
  (fp_line (start -1.27 -3.81) (end 1.27 -3.81) (layer F.SilkS) (width 0.15))
  (fp_line (start 1.27 -3.81) (end 1.27 3.81) (layer F.SilkS) (width 0.15))
  (fp_line (start 1.27 3.81) (end -1.27 3.81) (layer F.SilkS) (width 0.15))
  (fp_line (start -1.27 3.81) (end -1.27 -3.81) (layer F.SilkS) (width 0.15))
  (pad 3 thru_hole rect (at 0 2.54) (size 1.524 1.524) (drill 0.889) (layers *.Cu *.Mask F.SilkS) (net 4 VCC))
  (pad 2 thru_hole rect (at 0 0) (size 1.524 1.524) (drill 0.889) (layers *.Cu *.Mask F.SilkS) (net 13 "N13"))
  (pad 1 thru_hole rect (at 0 -2.54) (size 1.524 1.524) (drill 0.889) (layers *.Cu *.Mask F.SilkS) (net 5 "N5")))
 (gr_line (start 0.254 -0.254) (end 0.254 -40.386) (angle 90) (layer Edge.Cuts) (width 0.1))
 (gr_line (start 30.226 -0.254) (end 0.254 -0.254) (angle 90) (layer Edge.Cuts) (width 0.1))
 (gr_line (start 30.226 -40.386) (end 30.226 -0.254) (angle 90) (layer Edge.Cuts) (width 0.1))
 (gr_line (start 0.254 -40.386) (end 30.226 -40.386) (angle 90) (layer Edge.Cuts) (width 0.1))
 (segment (start 8.59282 -28.956) (end 8.59282 -28.30195) (width 0.254) (layer B.Cu) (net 1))
 (segment (start 8.59282 -28.30195) (end 9.20877 -27.686) (width 0.254) (layer B.Cu) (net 1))
 (segment (start 9.20877 -27.686) (end 9.9695 -27.686) (width 0.254) (layer B.Cu) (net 1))
 (segment (start 9.9695 -27.686) (end 10.9855 -27.686) (width 0.254) (layer B.Cu) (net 1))
 (segment (start 18.288 -16.1925) (end 20.828 -16.1925) (width 0.5) (layer B.Cu) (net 2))
 (segment (start 20.828 -16.1925) (end 20.8915 -16.256) (width 0.5) (layer B.Cu) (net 2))
 (segment (start 14.9305 -24.612) (end 14.9305 -22.853178) (width 0.254) (layer B.Cu) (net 2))
 (segment (start 14.9305 -22.853178) (end 16.447678 -21.336) (width 0.254) (layer B.Cu) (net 2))
 (segment (start 16.447678 -21.336) (end 16.59382 -21.336) (width 0.254) (layer B.Cu) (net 2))
 (segment (start 16.59382 -21.336) (end 17.49806 -21.336) (width 0.254) (layer B.Cu) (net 2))
 (segment (start 17.49806 -18.542) (end 17.49806 -21.336) (width 0.5) (layer B.Cu) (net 2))
 (segment (start 18.288 -16.1925) (end 18.288 -17.75206) (width 0.5) (layer B.Cu) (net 2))
 (segment (start 18.288 -17.75206) (end 17.49806 -18.542) (width 0.5) (layer B.Cu) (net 2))
 (segment (start 10.6045 -16.256) (end 13.1445 -16.256) (width 0.5) (layer B.Cu) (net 3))
 (segment (start 13.1445 -16.256) (end 13.208 -16.1925) (width 0.5) (layer B.Cu) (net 3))
 (segment (start 14.4305 -24.612) (end 14.4305 -21.76856) (width 0.254) (layer B.Cu) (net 3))
 (segment (start 14.4305 -21.76856) (end 13.99794 -21.336) (width 0.254) (layer B.Cu) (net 3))
 (segment (start 13.99794 -18.542) (end 13.99794 -21.336) (width 0.5) (layer B.Cu) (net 3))
 (segment (start 13.208 -16.1925) (end 13.208 -17.75206) (width 0.5) (layer B.Cu) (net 3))
 (segment (start 13.208 -17.75206) (end 13.99794 -18.542) (width 0.5) (layer B.Cu) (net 3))
 (segment (start 3.8735 -24.765) (end 6.35 -24.765) (width 0.254) (layer B.Cu) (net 4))
 (segment (start 6.35 -24.765) (end 6.5405 -24.5745) (width 0.254) (layer B.Cu) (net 4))
 (segment (start 16.508822 -23.5585) (end 16.891 -23.5585) (width 0.4) (layer B.Cu) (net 4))
 (segment (start 16.891 -23.5585) (end 18.034 -24.7015) (width 0.4) (layer B.Cu) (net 4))
 (segment (start 18.034 -24.7015) (end 18.288 -24.7015) (width 0.4) (layer B.Cu) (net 4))
 (segment (start 15.9305 -24.612) (end 15.9305 -24.136822) (width 0.254) (layer B.Cu) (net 4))
 (segment (start 15.9305 -24.136822) (end 16.508822 -23.5585) (width 0.254) (layer B.Cu) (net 4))
 (segment (start 18.288 -24.7015) (end 20.828 -24.7015) (width 0.4) (layer B.Cu) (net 4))
 (segment (start 6.39318 -28.0035) (end 6.39318 -29.9085) (width 0.254) (layer B.Cu) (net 5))
 (segment (start 3.8735 -29.845) (end 6.32968 -29.845) (width 0.254) (layer B.Cu) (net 5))
 (segment (start 6.32968 -29.845) (end 6.39318 -29.9085) (width 0.254) (layer B.Cu) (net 5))
 (segment (start 20.0025 -22.0345) (end 16.891 -22.0345) (width 0.3) (layer F.Cu) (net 6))
 (segment (start 16.891 -22.0345) (end 15.748 -23.1775) (width 0.3) (layer F.Cu) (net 6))
 (segment (start 15.4305 -24.612) (end 15.4305 -23.495) (width 0.254) (layer B.Cu) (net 6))
 (segment (start 15.4305 -23.495) (end 15.748 -23.1775) (width 0.254) (layer B.Cu) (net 6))
 (via (at 15.748 -23.1775) (size 0.889) (drill 0.635) (layers F.Cu B.Cu) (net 6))
 (segment (start 19.45001 -22.58699) (end 20.0025 -22.0345) (width 0.3) (layer F.Cu) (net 6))
 (segment (start 19.6215 -25.5905) (end 18.976999 -26.235001) (width 0.254) (layer F.Cu) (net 13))
 (segment (start 18.976999 -26.235001) (end 5.959499 -26.235001) (width 0.254) (layer F.Cu) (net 13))
 (segment (start 5.959499 -26.235001) (end 4.8895 -27.305) (width 0.254) (layer F.Cu) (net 13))
 (segment (start 4.8895 -27.305) (end 3.8735 -27.305) (width 0.254) (layer F.Cu) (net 13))
 (segment (start 16.4305 -24.612) (end 17.291501 -25.473001) (width 0.254) (layer B.Cu) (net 13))
 (segment (start 17.291501 -25.473001) (end 19.504001 -25.473001) (width 0.254) (layer B.Cu) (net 13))
 (segment (start 19.504001 -25.473001) (end 19.6215 -25.5905) (width 0.254) (layer B.Cu) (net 13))
 (via (at 19.6215 -25.5905) (size 0.889) (drill 0.635) (layers F.Cu B.Cu) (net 13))
 (segment (start 16.4305 -27.712) (end 23.088 -27.712) (width 0.254) (layer B.Cu) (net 7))
 (segment (start 23.088 -27.712) (end 23.876 -26.924) (width 0.254) (layer B.Cu) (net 7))
 (segment (start 15.9305 -27.712) (end 15.9305 -28.275602) (width 0.254) (layer B.Cu) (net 8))
 (segment (start 15.9305 -28.275602) (end 17.118898 -29.464) (width 0.254) (layer B.Cu) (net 8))
 (segment (start 17.118898 -29.464) (end 22.86 -29.464) (width 0.254) (layer B.Cu) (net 8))
 (segment (start 22.86 -29.464) (end 23.876 -29.464) (width 0.254) (layer B.Cu) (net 8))
 (segment (start 14.9305 -27.712) (end 14.9305 -28.291) (width 0.254) (layer B.Cu) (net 9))
 (segment (start 14.9305 -28.291) (end 16.675 -30.0355) (width 0.254) (layer B.Cu) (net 9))
 (segment (start 17.018 -30.0355) (end 17.7165 -30.734) (width 0.254) (layer B.Cu) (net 9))
 (segment (start 16.675 -30.0355) (end 17.018 -30.0355) (width 0.254) (layer B.Cu) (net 9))
 (segment (start 17.7165 -30.734) (end 17.7165 -30.988) (width 0.254) (layer B.Cu) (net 9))
 (segment (start 14.4305 -27.712) (end 14.4305 -28.8765) (width 0.254) (layer B.Cu) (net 10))
 (segment (start 14.4305 -28.8765) (end 13.2715 -30.0355) (width 0.254) (layer B.Cu) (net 10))
 (segment (start 13.2715 -30.0355) (end 13.0175 -30.0355) (width 0.254) (layer B.Cu) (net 10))
 (segment (start 13.0175 -30.0355) (end 12.319 -30.734) (width 0.254) (layer B.Cu) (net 10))
 (segment (start 12.319 -30.734) (end 12.319 -30.988) (width 0.254) (layer B.Cu) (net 10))
 (segment (start 18.288 -10.414) (end 18.288 -14.2875) (width 0.5) (layer B.Cu) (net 11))
 (segment (start 18.288 -5.414) (end 18.288 -7.819) (width 0.5) (layer B.Cu) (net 11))
 (segment (start 18.288 -7.819) (end 18.288 -10.414) (width 0.5) (layer B.Cu) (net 11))
 (segment (start 13.208 -10.414) (end 13.208 -14.2875) (width 0.5) (layer B.Cu) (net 12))
 (segment (start 13.208 -5.414) (end 13.208 -7.819) (width 0.5) (layer B.Cu) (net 12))
 (segment (start 13.208 -7.819) (end 13.208 -10.414) (width 0.5) (layer B.Cu) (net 12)))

